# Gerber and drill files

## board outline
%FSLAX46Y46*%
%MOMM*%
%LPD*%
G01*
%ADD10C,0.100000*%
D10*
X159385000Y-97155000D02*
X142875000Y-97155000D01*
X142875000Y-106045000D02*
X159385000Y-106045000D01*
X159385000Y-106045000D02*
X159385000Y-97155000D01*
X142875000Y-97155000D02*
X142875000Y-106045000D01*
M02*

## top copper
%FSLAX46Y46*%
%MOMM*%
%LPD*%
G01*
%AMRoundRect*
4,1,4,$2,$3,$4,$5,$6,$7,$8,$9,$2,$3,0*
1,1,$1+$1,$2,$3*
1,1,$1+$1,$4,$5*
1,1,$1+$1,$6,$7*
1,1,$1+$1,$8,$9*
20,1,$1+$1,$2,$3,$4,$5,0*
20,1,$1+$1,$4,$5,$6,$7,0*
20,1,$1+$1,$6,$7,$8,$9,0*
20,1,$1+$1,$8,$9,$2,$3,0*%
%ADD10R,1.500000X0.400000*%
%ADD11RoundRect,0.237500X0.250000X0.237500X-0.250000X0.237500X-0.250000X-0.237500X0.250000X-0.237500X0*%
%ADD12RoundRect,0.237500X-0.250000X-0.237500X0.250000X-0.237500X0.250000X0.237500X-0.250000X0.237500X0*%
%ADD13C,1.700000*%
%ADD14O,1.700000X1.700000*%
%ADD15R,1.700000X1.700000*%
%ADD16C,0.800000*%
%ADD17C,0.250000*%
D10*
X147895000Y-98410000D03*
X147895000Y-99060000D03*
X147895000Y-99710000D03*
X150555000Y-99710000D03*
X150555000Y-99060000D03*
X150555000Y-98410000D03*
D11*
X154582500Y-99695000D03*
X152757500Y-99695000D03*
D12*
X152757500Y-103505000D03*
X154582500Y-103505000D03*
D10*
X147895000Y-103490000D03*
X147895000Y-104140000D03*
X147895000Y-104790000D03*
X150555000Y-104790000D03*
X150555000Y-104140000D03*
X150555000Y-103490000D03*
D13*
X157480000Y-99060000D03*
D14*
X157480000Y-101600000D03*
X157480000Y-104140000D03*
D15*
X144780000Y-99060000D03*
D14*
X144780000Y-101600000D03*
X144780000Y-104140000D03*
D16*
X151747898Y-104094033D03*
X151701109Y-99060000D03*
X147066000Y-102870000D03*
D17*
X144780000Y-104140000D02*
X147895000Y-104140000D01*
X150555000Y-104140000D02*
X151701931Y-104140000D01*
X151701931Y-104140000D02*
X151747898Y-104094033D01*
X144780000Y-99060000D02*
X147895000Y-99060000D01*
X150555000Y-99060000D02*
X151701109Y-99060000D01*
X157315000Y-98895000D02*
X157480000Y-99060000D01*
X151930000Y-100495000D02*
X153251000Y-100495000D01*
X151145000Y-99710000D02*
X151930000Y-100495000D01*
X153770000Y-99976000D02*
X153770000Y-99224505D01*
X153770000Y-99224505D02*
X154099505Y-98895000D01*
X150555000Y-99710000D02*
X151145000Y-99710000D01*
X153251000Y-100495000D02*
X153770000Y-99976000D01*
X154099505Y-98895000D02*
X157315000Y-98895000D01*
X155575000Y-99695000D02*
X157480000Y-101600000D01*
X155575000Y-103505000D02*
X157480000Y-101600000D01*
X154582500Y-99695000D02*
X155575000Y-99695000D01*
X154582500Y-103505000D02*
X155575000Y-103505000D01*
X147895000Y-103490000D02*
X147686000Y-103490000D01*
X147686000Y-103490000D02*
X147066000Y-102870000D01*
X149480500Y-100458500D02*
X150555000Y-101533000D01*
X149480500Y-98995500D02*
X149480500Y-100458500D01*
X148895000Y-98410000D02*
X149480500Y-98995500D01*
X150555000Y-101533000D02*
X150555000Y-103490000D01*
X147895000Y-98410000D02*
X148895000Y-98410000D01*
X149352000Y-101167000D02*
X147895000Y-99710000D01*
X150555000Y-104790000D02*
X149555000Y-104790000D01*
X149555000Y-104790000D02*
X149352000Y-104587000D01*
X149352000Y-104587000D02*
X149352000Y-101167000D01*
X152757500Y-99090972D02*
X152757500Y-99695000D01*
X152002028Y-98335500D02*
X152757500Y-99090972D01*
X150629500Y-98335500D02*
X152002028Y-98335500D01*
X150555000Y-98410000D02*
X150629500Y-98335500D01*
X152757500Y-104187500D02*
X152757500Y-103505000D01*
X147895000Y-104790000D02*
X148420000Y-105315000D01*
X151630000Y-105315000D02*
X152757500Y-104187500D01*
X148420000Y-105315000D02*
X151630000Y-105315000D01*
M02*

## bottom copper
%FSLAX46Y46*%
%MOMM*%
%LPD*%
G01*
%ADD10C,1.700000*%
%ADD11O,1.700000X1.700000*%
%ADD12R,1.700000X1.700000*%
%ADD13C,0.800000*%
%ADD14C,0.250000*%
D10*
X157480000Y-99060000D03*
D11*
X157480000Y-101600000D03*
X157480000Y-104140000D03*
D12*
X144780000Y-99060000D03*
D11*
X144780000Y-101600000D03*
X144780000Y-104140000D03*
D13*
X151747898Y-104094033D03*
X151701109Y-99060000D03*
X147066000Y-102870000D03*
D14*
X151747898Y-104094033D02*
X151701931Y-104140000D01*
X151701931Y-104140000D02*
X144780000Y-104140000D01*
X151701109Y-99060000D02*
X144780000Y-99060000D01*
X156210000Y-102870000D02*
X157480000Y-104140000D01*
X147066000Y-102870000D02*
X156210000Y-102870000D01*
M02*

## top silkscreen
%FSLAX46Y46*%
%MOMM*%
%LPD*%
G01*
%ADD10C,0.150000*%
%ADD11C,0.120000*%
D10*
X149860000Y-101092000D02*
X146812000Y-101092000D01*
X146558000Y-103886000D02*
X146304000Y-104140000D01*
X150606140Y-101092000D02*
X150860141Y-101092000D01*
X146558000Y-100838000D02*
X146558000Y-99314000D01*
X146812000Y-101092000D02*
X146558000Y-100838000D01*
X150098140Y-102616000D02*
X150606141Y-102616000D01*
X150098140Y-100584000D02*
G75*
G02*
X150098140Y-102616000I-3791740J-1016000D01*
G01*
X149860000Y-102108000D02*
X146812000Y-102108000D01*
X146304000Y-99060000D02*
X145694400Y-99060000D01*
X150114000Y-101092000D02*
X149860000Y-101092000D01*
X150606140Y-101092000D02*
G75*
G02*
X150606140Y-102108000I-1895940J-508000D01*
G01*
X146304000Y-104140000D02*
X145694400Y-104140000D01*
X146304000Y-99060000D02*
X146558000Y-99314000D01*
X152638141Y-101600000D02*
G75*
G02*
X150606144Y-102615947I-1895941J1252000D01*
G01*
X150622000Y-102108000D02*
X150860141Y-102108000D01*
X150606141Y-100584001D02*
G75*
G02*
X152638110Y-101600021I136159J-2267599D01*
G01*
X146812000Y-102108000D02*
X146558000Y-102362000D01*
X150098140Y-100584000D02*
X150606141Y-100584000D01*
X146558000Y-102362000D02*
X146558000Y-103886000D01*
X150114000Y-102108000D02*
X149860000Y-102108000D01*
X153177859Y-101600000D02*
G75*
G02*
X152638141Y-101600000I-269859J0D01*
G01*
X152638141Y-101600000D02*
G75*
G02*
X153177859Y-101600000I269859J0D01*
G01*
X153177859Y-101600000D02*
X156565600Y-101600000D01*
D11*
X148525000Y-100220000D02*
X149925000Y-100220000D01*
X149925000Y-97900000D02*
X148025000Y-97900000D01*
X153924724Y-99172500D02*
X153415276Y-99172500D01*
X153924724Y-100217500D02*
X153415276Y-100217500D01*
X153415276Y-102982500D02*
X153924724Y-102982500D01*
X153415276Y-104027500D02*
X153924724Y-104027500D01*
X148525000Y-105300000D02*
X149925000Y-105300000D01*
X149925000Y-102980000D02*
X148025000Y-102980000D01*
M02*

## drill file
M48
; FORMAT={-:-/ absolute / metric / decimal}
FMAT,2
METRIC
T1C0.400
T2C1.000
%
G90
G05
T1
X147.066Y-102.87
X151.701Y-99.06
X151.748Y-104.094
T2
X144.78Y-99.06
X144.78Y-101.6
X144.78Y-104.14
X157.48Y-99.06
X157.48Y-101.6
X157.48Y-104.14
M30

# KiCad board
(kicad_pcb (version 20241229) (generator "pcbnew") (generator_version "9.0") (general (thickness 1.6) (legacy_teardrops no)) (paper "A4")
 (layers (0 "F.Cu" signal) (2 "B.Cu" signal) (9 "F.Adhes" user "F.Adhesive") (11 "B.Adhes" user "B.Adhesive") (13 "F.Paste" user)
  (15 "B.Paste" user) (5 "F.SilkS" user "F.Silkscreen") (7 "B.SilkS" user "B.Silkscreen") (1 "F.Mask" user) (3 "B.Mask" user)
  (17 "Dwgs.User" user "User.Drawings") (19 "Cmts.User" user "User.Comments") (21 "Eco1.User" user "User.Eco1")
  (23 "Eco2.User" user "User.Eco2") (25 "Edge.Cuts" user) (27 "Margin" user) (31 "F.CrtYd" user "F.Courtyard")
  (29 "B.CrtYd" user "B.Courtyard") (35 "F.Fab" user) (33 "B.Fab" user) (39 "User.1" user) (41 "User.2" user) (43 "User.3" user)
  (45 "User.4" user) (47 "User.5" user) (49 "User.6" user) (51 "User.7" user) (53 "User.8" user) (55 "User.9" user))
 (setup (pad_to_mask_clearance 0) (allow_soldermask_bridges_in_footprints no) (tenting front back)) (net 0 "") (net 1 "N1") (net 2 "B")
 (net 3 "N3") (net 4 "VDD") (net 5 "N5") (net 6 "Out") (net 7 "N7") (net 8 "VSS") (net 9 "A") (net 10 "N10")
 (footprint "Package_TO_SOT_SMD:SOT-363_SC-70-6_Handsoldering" (layer "F.Cu") (at 149.225 99.06)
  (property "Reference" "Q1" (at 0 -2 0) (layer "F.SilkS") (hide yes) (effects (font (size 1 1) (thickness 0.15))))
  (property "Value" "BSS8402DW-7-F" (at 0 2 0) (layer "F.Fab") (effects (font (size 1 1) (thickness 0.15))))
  (fp_line (start -0.7 1.16) (end 0.7 1.16) (stroke (width 0.12) (type solid)) (layer "F.SilkS"))
  (fp_line (start 0.7 -1.16) (end -1.2 -1.16) (stroke (width 0.12) (type solid)) (layer "F.SilkS"))
  (pad "1" smd rect (at -1.33 -0.65) (size 1.5 0.4) (layers "F.Cu" "F.Mask" "F.Paste") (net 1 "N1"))
  (pad "2" smd rect (at -1.33 0) (size 1.5 0.4) (layers "F.Cu" "F.Mask" "F.Paste") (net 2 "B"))
  (pad "3" smd rect (at -1.33 0.65) (size 1.5 0.4) (layers "F.Cu" "F.Mask" "F.Paste") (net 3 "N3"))
  (pad "4" smd rect (at 1.33 0.65) (size 1.5 0.4) (layers "F.Cu" "F.Mask" "F.Paste") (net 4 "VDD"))
  (pad "5" smd rect (at 1.33 0) (size 1.5 0.4) (layers "F.Cu" "F.Mask" "F.Paste") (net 2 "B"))
  (pad "6" smd rect (at 1.33 -0.65) (size 1.5 0.4) (layers "F.Cu" "F.Mask" "F.Paste") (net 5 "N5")))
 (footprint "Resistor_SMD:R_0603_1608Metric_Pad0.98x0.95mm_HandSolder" (layer "F.Cu") (at 153.67 99.695 180)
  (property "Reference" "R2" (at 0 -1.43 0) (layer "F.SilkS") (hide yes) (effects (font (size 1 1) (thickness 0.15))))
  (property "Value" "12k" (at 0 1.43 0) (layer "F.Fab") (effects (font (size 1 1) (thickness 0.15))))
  (fp_line (start -0.254724 0.5225) (end 0.254724 0.5225) (stroke (width 0.12) (type solid)) (layer "F.SilkS"))
  (fp_line (start -0.254724 -0.5225) (end 0.254724 -0.5225) (stroke (width 0.12) (type solid)) (layer "F.SilkS"))
  (pad "1" smd roundrect (at -0.9125 0 180) (size 0.975 0.95) (layers "F.Cu" "F.Mask" "F.Paste") (roundrect_rratio 0.25) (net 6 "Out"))
  (pad "2" smd roundrect (at 0.9125 0 180) (size 0.975 0.95) (layers "F.Cu" "F.Mask" "F.Paste") (roundrect_rratio 0.25) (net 5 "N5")))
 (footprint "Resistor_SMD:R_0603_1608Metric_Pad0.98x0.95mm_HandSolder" (layer "F.Cu") (at 153.67 103.505)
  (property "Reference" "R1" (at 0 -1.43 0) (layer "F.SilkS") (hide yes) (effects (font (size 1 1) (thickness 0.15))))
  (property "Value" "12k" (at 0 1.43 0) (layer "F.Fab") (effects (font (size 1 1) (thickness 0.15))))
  (fp_line (start -0.254724 -0.5225) (end 0.254724 -0.5225) (stroke (width 0.12) (type solid)) (layer "F.SilkS"))
  (fp_line (start -0.254724 0.5225) (end 0.254724 0.5225) (stroke (width 0.12) (type solid)) (layer "F.SilkS"))
  (pad "1" smd roundrect (at -0.9125 0) (size 0.975 0.95) (layers "F.Cu" "F.Mask" "F.Paste") (roundrect_rratio 0.25) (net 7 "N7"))
  (pad "2" smd roundrect (at 0.9125 0) (size 0.975 0.95) (layers "F.Cu" "F.Mask" "F.Paste") (roundrect_rratio 0.25) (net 6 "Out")))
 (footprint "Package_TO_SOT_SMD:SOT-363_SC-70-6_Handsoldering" (layer "F.Cu") (at 149.225 104.14)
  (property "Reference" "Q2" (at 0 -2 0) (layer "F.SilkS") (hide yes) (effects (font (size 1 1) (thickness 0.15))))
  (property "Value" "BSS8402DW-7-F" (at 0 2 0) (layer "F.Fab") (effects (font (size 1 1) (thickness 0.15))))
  (fp_line (start -0.7 1.16) (end 0.7 1.16) (stroke (width 0.12) (type solid)) (layer "F.SilkS"))
  (fp_line (start 0.7 -1.16) (end -1.2 -1.16) (stroke (width 0.12) (type solid)) (layer "F.SilkS"))
  (pad "1" smd rect (at -1.33 -0.65) (size 1.5 0.4) (layers "F.Cu" "F.Mask" "F.Paste") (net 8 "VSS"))
  (pad "2" smd rect (at -1.33 0) (size 1.5 0.4) (layers "F.Cu" "F.Mask" "F.Paste") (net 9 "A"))
  (pad "3" smd rect (at -1.33 0.65) (size 1.5 0.4) (layers "F.Cu" "F.Mask" "F.Paste") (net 7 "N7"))
  (pad "4" smd rect (at 1.33 0.65) (size 1.5 0.4) (layers "F.Cu" "F.Mask" "F.Paste") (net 3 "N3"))
  (pad "5" smd rect (at 1.33 0) (size 1.5 0.4) (layers "F.Cu" "F.Mask" "F.Paste") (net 9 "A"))
  (pad "6" smd rect (at 1.33 -0.65) (size 1.5 0.4) (layers "F.Cu" "F.Mask" "F.Paste") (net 1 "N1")))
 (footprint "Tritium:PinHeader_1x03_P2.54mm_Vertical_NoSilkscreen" (layer "F.Cu") (at 157.48 99.06)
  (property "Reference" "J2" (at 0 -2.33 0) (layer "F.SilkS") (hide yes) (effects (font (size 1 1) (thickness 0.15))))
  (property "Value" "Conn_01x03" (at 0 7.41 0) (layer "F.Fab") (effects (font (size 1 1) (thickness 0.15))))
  (pad "1" thru_hole circle (at 0 0) (size 1.7 1.7) (drill 1) (layers "*.Cu" "*.Mask") (remove_unused_layers no) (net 4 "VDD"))
  (pad "2" thru_hole oval (at 0 2.54) (size 1.7 1.7) (drill 1) (layers "*.Cu" "*.Mask") (remove_unused_layers no) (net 6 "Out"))
  (pad "3" thru_hole oval (at 0 5.08) (size 1.7 1.7) (drill 1) (layers "*.Cu" "*.Mask") (remove_unused_layers no) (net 8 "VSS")))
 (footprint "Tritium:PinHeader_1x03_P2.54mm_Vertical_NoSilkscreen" (layer "F.Cu") (at 144.78 99.06)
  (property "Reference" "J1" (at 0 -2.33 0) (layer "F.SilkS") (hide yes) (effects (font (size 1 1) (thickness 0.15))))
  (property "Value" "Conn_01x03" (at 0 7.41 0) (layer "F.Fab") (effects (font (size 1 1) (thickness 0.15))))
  (pad "1" thru_hole rect (at 0 0) (size 1.7 1.7) (drill 1) (layers "*.Cu" "*.Mask") (remove_unused_layers no) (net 2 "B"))
  (pad "2" thru_hole oval (at 0 2.54) (size 1.7 1.7) (drill 1) (layers "*.Cu" "*.Mask") (remove_unused_layers no) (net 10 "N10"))
  (pad "3" thru_hole oval (at 0 5.08) (size 1.7 1.7) (drill 1) (layers "*.Cu" "*.Mask") (remove_unused_layers no) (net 9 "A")))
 (gr_line (start 149.86 101.092) (end 146.812 101.092) (stroke (width 0.15) (type solid)) (layer "F.SilkS"))
 (gr_line (start 146.558 103.886) (end 146.304 104.14) (stroke (width 0.15) (type solid)) (layer "F.SilkS"))
 (gr_line (start 150.60614 101.092) (end 150.860141 101.092) (stroke (width 0.15) (type solid)) (layer "F.SilkS"))
 (gr_line (start 146.558 100.838) (end 146.558 99.314) (stroke (width 0.15) (type solid)) (layer "F.SilkS"))
 (gr_line (start 146.812 101.092) (end 146.558 100.838) (stroke (width 0.15) (type solid)) (layer "F.SilkS"))
 (gr_line (start 150.09814 102.616) (end 150.606141 102.616) (stroke (width 0.15) (type solid)) (layer "F.SilkS"))
 (gr_arc (start 150.09814 100.584) (mid 150.2319 101.6) (end 150.09814 102.616) (stroke (width 0.15) (type solid)) (layer "F.SilkS"))
 (gr_line (start 149.86 102.108) (end 146.812 102.108) (stroke (width 0.15) (type solid)) (layer "F.SilkS"))
 (gr_line (start 146.304 99.06) (end 145.6944 99.06) (stroke (width 0.15) (type solid)) (layer "F.SilkS"))
 (gr_line (start 150.114 101.092) (end 149.86 101.092) (stroke (width 0.15) (type solid)) (layer "F.SilkS"))
 (gr_arc (start 150.60614 101.092) (mid 150.673017 101.6) (end 150.60614 102.108) (stroke (width 0.15) (type solid)) (layer "F.SilkS"))
 (gr_line (start 146.304 104.14) (end 145.6944 104.14) (stroke (width 0.15) (type solid)) (layer "F.SilkS"))
 (gr_line (start 146.304 99.06) (end 146.558 99.314) (stroke (width 0.15) (type solid)) (layer "F.SilkS"))
 (gr_arc (start 152.638141 101.6) (mid 151.758253 102.380208) (end 150.606141 102.616) (stroke (width 0.15) (type solid)) (layer "F.SilkS"))
 (gr_line (start 150.622 102.108) (end 150.860141 102.108) (stroke (width 0.15) (type solid)) (layer "F.SilkS"))
 (gr_arc (start 150.606141 100.584001) (mid 151.758276 100.819746) (end 152.638141 101.6) (stroke (width 0.15) (type solid))
  (layer "F.SilkS"))
 (gr_line (start 146.812 102.108) (end 146.558 102.362) (stroke (width 0.15) (type solid)) (layer "F.SilkS"))
 (gr_line (start 150.09814 100.584) (end 150.606141 100.584) (stroke (width 0.15) (type solid)) (layer "F.SilkS"))
 (gr_line (start 146.558 102.362) (end 146.558 103.886) (stroke (width 0.15) (type solid)) (layer "F.SilkS"))
 (gr_line (start 150.114 102.108) (end 149.86 102.108) (stroke (width 0.15) (type solid)) (layer "F.SilkS"))
 (gr_circle (center 152.908 101.6) (end 152.638141 101.6) (stroke (width 0.15) (type solid)) (fill no) (layer "F.SilkS"))
 (gr_line (start 153.177859 101.6) (end 156.5656 101.6) (stroke (width 0.15) (type solid)) (layer "F.SilkS"))
 (gr_line (start 159.385 97.155) (end 142.875 97.155) (stroke (width 0.1) (type solid)) (layer "Edge.Cuts"))
 (gr_line (start 142.875 106.045) (end 159.385 106.045) (stroke (width 0.1) (type solid)) (layer "Edge.Cuts"))
 (gr_line (start 159.385 106.045) (end 159.385 97.155) (stroke (width 0.1) (type solid)) (layer "Edge.Cuts"))
 (gr_line (start 142.875 97.155) (end 142.875 106.045) (stroke (width 0.1) (type solid)) (layer "Edge.Cuts"))
 (segment (start 144.78 104.14) (end 147.895 104.14) (width 0.25) (layer "F.Cu") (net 9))
 (segment (start 150.555 104.14) (end 151.701931 104.14) (width 0.25) (layer "F.Cu") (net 9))
 (segment (start 151.701931 104.14) (end 151.747898 104.094033) (width 0.25) (layer "F.Cu") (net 9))
 (via (at 151.747898 104.094033) (size 0.8) (drill 0.4) (layers "F.Cu" "B.Cu") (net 9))
 (segment (start 151.747898 104.094033) (end 151.701931 104.14) (width 0.25) (layer "B.Cu") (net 9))
 (segment (start 151.701931 104.14) (end 144.78 104.14) (width 0.25) (layer "B.Cu") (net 9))
 (segment (start 144.78 99.06) (end 147.895 99.06) (width 0.25) (layer "F.Cu") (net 2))
 (segment (start 150.555 99.06) (end 151.701109 99.06) (width 0.25) (layer "F.Cu") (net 2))
 (via (at 151.701109 99.06) (size 0.8) (drill 0.4) (layers "F.Cu" "B.Cu") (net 2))
 (segment (start 151.701109 99.06) (end 144.78 99.06) (width 0.25) (layer "B.Cu") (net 2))
 (segment (start 157.315 98.895) (end 157.48 99.06) (width 0.25) (layer "F.Cu") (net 4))
 (segment (start 151.93 100.495) (end 153.251 100.495) (width 0.25) (layer "F.Cu") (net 4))
 (segment (start 151.145 99.71) (end 151.93 100.495) (width 0.25) (layer "F.Cu") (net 4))
 (segment (start 153.77 99.976) (end 153.77 99.224505) (width 0.25) (layer "F.Cu") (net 4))
 (segment (start 153.77 99.224505) (end 154.099505 98.895) (width 0.25) (layer "F.Cu") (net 4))
 (segment (start 150.555 99.71) (end 151.145 99.71) (width 0.25) (layer "F.Cu") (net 4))
 (segment (start 153.251 100.495) (end 153.77 99.976) (width 0.25) (layer "F.Cu") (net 4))
 (segment (start 154.099505 98.895) (end 157.315 98.895) (width 0.25) (layer "F.Cu") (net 4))
 (segment (start 155.575 99.695) (end 157.48 101.6) (width 0.25) (layer "F.Cu") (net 6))
 (segment (start 155.575 103.505) (end 157.48 101.6) (width 0.25) (layer "F.Cu") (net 6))
 (segment (start 154.5825 99.695) (end 155.575 99.695) (width 0.25) (layer "F.Cu") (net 6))
 (segment (start 154.5825 103.505) (end 155.575 103.505) (width 0.25) (layer "F.Cu") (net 6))
 (segment (start 147.895 103.49) (end 147.686 103.49) (width 0.25) (layer "F.Cu") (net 8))
 (segment (start 147.686 103.49) (end 147.066 102.87) (width 0.25) (layer "F.Cu") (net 8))
 (via (at 147.066 102.87) (size 0.8) (drill 0.4) (layers "F.Cu" "B.Cu") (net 8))
 (segment (start 156.21 102.87) (end 157.48 104.14) (width 0.25) (layer "B.Cu") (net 8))
 (segment (start 147.066 102.87) (end 156.21 102.87) (width 0.25) (layer "B.Cu") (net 8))
 (segment (start 149.4805 100.4585) (end 150.555 101.533) (width 0.25) (layer "F.Cu") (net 1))
 (segment (start 149.4805 98.9955) (end 149.4805 100.4585) (width 0.25) (layer "F.Cu") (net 1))
 (segment (start 148.895 98.41) (end 149.4805 98.9955) (width 0.25) (layer "F.Cu") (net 1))
 (segment (start 150.555 101.533) (end 150.555 103.49) (width 0.25) (layer "F.Cu") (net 1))
 (segment (start 147.895 98.41) (end 148.895 98.41) (width 0.25) (layer "F.Cu") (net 1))
 (segment (start 149.352 101.167) (end 147.895 99.71) (width 0.25) (layer "F.Cu") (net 3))
 (segment (start 150.555 104.79) (end 149.555 104.79) (width 0.25) (layer "F.Cu") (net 3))
 (segment (start 149.555 104.79) (end 149.352 104.587) (width 0.25) (layer "F.Cu") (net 3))
 (segment (start 149.352 104.587) (end 149.352 101.167) (width 0.25) (layer "F.Cu") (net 3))
 (segment (start 152.7575 99.090972) (end 152.7575 99.695) (width 0.25) (layer "F.Cu") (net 5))
 (segment (start 152.002028 98.3355) (end 152.7575 99.090972) (width 0.25) (layer "F.Cu") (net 5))
 (segment (start 150.6295 98.3355) (end 152.002028 98.3355) (width 0.25) (layer "F.Cu") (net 5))
 (segment (start 150.555 98.41) (end 150.6295 98.3355) (width 0.25) (layer "F.Cu") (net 5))
 (segment (start 152.7575 104.1875) (end 152.7575 103.505) (width 0.25) (layer "F.Cu") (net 7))
 (segment (start 147.895 104.79) (end 148.42 105.315) (width 0.25) (layer "F.Cu") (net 7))
 (segment (start 151.63 105.315) (end 152.7575 104.1875) (width 0.25) (layer "F.Cu") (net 7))
 (segment (start 148.42 105.315) (end 151.63 105.315) (width 0.25) (layer "F.Cu") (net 7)))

